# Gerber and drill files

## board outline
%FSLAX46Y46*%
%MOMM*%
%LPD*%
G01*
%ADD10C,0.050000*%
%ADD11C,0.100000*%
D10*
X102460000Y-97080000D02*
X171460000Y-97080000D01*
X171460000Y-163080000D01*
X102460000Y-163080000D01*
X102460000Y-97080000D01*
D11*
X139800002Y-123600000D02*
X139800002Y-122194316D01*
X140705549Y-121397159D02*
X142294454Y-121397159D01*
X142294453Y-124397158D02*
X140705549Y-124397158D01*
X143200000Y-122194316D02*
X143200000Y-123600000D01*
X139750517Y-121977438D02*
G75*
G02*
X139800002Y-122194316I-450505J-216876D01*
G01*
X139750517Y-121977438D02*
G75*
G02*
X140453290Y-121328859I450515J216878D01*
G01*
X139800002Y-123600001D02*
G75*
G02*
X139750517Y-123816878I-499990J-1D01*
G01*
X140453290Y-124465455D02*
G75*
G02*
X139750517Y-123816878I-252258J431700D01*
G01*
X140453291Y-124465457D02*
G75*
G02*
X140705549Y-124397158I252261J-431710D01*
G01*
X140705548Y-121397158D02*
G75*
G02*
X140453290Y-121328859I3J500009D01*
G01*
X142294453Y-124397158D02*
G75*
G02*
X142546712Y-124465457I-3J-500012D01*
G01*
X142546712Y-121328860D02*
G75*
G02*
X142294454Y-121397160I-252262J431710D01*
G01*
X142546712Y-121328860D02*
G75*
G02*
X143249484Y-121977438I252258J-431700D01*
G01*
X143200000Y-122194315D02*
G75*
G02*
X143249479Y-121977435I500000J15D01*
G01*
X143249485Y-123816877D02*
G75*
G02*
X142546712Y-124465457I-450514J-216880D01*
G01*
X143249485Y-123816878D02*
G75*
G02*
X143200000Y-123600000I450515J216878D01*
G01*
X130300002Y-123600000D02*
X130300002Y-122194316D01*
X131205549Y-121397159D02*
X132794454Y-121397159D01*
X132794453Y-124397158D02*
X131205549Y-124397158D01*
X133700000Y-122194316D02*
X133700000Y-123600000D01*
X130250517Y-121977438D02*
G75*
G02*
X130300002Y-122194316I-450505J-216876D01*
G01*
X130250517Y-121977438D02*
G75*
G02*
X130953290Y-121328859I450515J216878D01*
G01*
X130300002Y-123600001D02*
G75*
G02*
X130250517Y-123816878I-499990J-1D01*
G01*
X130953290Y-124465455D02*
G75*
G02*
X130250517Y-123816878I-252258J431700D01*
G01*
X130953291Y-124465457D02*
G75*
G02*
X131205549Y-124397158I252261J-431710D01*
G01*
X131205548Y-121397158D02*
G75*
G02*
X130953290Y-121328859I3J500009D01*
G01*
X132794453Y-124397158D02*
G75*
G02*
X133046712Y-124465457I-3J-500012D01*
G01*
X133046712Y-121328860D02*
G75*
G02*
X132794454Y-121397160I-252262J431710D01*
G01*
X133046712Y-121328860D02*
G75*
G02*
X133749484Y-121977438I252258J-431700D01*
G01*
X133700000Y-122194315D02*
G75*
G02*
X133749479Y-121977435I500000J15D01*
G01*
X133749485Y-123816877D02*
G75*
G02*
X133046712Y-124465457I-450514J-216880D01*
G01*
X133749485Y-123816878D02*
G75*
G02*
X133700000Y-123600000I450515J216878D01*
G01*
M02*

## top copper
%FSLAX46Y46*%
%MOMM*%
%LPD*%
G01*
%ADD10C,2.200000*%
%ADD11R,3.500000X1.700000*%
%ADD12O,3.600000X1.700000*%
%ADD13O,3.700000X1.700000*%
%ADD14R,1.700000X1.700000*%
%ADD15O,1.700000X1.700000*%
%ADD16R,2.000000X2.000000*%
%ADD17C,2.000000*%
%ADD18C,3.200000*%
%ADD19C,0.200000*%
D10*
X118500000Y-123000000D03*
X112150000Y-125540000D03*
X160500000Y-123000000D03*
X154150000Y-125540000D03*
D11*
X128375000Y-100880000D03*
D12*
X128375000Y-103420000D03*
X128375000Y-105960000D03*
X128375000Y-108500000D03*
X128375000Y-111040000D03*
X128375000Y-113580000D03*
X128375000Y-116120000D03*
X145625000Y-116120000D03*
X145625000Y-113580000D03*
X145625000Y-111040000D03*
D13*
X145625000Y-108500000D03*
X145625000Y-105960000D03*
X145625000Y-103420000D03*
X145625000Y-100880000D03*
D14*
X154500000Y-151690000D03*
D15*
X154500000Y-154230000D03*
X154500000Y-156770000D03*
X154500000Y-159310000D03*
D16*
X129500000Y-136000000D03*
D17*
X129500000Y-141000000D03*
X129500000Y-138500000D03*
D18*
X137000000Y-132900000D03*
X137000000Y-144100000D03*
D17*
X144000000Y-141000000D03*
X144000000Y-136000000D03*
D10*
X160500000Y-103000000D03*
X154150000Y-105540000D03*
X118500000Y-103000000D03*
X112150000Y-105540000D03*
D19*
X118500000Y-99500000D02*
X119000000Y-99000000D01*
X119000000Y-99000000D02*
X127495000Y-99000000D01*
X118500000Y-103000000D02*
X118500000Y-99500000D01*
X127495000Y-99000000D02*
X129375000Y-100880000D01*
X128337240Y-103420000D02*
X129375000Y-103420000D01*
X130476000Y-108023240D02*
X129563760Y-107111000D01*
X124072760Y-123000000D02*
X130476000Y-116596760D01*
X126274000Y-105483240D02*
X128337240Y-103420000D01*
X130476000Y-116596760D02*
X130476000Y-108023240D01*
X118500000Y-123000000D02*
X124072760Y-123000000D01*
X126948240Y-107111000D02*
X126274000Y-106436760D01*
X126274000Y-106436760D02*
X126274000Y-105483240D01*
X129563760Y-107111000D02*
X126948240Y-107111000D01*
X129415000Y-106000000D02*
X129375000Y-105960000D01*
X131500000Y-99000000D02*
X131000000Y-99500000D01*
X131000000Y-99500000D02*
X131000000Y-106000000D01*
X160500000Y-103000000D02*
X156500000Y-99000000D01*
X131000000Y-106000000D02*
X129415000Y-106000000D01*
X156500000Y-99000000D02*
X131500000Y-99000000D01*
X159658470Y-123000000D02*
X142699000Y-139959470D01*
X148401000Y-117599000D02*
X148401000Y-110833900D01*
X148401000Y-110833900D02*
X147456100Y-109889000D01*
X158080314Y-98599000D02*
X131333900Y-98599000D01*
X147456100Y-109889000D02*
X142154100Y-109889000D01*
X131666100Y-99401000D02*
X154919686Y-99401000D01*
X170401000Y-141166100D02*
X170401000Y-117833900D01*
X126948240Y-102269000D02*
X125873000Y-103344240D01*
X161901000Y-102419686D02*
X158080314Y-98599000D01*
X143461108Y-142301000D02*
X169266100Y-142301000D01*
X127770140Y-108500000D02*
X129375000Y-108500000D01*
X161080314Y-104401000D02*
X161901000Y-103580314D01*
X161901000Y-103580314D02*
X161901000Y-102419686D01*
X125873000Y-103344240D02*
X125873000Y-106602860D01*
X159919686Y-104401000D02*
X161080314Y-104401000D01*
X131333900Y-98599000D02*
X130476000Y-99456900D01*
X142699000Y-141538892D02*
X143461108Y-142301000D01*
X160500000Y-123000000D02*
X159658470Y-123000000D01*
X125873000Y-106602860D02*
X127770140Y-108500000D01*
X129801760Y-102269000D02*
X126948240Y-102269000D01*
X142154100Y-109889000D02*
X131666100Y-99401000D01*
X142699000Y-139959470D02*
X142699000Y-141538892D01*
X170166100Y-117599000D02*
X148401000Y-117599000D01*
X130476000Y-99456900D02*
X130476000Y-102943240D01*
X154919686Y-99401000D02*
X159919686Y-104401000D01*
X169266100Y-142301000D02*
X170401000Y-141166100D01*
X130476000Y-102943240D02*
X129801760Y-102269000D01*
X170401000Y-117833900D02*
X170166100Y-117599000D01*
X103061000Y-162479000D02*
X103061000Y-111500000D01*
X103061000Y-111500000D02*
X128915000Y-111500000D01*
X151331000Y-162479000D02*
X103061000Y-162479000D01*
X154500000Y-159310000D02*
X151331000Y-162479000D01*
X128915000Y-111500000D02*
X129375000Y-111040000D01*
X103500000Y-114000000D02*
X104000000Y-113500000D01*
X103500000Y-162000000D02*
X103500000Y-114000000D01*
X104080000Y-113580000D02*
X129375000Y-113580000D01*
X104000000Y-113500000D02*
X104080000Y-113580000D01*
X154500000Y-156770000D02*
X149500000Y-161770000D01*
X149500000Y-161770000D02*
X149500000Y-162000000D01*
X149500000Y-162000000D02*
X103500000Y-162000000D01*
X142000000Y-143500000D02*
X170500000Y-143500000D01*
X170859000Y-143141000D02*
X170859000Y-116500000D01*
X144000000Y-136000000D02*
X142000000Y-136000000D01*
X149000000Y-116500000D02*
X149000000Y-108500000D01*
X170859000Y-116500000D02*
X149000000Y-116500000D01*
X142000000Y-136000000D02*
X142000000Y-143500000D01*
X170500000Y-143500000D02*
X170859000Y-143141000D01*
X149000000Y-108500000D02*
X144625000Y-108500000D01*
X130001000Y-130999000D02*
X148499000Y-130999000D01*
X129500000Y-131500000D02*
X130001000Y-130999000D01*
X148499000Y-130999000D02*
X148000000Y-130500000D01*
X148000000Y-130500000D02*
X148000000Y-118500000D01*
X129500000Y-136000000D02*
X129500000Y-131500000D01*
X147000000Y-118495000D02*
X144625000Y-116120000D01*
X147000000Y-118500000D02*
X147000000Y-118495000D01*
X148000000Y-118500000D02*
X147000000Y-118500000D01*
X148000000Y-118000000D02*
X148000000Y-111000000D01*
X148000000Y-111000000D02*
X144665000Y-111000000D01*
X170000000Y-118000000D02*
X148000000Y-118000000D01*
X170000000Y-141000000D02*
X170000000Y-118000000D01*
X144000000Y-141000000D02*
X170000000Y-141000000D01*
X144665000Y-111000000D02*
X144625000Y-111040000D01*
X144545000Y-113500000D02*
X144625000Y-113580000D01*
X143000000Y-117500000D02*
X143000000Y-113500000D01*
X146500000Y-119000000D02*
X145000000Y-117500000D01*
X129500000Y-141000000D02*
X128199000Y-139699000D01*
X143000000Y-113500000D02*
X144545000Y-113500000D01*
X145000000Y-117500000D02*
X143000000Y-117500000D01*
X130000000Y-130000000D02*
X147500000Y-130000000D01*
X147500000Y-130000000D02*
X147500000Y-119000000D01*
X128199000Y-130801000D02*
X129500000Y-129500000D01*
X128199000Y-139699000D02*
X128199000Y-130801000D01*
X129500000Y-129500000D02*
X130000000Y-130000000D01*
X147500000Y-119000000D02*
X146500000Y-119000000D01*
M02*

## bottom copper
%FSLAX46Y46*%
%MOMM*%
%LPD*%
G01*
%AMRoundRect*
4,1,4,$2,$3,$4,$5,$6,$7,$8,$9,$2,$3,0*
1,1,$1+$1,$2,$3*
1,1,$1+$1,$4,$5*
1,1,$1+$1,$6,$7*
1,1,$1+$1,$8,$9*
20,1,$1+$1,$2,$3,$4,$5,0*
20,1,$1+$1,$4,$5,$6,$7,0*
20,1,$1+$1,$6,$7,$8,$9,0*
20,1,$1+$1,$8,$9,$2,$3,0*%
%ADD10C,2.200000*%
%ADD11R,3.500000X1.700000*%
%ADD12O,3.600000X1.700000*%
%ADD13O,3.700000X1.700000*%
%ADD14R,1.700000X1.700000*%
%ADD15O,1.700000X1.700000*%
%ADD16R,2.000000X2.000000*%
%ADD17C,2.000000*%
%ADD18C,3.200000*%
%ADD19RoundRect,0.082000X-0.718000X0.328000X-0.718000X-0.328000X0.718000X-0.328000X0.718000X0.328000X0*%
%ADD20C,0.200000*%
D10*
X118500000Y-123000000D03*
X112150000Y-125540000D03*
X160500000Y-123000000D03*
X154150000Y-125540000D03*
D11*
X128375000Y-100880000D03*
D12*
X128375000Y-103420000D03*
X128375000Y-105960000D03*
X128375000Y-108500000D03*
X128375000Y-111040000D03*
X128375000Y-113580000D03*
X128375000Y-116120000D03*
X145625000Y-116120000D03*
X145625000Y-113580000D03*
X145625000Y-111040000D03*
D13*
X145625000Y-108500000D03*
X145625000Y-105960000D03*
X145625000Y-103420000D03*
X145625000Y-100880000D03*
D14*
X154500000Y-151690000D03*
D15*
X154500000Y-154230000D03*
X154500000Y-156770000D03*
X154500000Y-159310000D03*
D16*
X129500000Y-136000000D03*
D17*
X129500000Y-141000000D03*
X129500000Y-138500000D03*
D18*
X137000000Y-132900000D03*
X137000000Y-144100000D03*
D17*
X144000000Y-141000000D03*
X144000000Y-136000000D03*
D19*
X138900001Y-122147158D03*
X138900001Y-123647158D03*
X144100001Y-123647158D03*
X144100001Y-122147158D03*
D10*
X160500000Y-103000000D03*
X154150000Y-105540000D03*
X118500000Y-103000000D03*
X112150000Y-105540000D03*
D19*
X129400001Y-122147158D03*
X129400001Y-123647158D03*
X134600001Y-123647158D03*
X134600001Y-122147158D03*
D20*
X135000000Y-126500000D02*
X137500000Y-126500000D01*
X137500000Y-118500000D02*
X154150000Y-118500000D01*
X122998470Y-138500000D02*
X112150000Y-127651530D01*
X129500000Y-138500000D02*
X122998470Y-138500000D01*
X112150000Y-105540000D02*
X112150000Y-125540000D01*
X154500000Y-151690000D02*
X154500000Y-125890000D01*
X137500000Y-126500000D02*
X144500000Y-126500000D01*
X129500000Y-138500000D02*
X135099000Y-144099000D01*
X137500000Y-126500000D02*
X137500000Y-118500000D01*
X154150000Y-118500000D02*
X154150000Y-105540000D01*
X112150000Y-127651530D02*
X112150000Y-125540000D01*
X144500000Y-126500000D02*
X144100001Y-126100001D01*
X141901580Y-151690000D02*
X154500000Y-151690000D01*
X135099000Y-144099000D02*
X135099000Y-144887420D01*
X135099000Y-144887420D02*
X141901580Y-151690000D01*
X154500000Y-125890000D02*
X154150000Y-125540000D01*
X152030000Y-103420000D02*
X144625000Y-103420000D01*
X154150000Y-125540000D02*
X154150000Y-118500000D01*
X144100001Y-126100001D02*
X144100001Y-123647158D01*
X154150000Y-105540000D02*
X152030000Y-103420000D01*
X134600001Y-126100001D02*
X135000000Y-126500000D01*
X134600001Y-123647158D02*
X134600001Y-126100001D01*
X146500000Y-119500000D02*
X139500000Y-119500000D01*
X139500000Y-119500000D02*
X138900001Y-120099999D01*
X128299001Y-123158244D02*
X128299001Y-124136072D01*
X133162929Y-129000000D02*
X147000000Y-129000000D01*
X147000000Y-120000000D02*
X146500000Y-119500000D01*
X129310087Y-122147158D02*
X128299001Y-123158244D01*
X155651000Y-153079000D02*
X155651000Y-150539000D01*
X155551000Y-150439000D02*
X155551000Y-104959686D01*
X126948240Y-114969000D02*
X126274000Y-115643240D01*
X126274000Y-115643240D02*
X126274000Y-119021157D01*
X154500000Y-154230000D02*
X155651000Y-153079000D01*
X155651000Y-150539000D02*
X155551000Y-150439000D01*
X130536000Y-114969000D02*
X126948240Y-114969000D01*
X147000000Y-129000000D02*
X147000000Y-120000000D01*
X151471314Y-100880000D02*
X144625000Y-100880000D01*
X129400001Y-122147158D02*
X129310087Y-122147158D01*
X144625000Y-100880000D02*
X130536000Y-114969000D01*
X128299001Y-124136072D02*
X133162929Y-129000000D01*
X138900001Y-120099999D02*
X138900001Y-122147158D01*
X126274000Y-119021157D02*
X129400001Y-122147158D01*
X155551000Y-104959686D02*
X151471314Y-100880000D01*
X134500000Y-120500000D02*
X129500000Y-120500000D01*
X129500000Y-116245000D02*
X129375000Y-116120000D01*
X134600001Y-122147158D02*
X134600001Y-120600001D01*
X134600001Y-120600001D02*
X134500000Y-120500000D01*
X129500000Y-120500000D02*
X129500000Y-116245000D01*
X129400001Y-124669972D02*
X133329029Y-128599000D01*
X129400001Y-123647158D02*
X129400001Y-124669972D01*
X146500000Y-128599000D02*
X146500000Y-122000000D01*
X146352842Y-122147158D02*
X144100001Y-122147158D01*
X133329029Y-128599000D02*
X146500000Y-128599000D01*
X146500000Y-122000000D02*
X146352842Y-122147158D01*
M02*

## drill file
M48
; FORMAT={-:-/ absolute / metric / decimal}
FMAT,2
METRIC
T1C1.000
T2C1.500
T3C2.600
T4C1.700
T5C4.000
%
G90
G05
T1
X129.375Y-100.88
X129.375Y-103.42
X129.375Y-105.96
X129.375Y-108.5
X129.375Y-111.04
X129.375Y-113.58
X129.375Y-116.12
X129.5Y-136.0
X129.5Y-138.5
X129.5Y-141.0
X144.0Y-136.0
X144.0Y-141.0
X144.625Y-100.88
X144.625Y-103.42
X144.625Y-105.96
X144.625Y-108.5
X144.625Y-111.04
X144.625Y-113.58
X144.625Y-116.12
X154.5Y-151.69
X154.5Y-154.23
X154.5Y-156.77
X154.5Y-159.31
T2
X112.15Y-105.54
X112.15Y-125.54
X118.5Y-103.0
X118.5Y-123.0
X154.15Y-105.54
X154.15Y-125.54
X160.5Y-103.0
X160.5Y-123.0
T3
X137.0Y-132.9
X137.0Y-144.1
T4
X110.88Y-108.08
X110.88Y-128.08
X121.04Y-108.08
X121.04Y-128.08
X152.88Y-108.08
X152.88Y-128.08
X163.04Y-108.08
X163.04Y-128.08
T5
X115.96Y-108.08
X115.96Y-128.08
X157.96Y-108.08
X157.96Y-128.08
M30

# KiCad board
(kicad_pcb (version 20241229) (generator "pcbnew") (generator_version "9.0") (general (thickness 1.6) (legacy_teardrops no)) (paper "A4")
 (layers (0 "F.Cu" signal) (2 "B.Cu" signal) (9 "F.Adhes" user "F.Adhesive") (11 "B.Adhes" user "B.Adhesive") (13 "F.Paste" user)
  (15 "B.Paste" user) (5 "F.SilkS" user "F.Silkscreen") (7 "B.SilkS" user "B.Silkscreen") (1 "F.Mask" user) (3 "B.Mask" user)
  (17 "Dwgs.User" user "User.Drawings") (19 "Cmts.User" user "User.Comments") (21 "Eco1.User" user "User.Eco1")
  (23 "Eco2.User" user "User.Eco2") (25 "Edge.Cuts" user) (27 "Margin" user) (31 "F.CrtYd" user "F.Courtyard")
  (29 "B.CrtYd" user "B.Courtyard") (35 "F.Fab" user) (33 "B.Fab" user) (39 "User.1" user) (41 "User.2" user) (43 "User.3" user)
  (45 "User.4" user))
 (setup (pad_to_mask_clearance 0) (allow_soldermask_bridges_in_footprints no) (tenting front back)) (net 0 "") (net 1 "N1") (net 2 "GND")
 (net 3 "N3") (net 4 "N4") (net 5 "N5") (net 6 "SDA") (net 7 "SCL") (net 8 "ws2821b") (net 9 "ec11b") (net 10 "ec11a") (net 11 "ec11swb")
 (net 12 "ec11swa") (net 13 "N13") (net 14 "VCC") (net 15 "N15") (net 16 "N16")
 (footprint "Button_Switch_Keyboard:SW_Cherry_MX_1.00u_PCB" (layer "F.Cu") (at 118.5 123)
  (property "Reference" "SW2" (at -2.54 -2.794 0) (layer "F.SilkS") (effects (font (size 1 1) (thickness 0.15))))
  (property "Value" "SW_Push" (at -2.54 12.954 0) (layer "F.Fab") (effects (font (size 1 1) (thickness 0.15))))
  (pad "" np_thru_hole circle (at -7.62 5.08) (size 1.7 1.7) (drill 1.7) (layers "*.Cu" "*.Mask"))
  (pad "" np_thru_hole circle (at -2.54 5.08) (size 4 4) (drill 4) (layers "*.Cu" "*.Mask"))
  (pad "" np_thru_hole circle (at 2.54 5.08) (size 1.7 1.7) (drill 1.7) (layers "*.Cu" "*.Mask"))
  (pad "1" thru_hole circle (at 0 0) (size 2.2 2.2) (drill 1.5) (layers "*.Cu" "*.Mask") (remove_unused_layers no) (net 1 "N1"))
  (pad "2" thru_hole circle (at -6.35 2.54) (size 2.2 2.2) (drill 1.5) (layers "*.Cu" "*.Mask") (remove_unused_layers no) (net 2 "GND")))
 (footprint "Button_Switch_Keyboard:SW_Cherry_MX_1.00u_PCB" (layer "F.Cu") (at 160.5 123)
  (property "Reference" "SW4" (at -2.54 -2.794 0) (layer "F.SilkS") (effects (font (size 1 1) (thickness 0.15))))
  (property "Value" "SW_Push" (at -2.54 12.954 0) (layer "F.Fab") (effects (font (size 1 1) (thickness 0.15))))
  (pad "" np_thru_hole circle (at -7.62 5.08) (size 1.7 1.7) (drill 1.7) (layers "*.Cu" "*.Mask"))
  (pad "" np_thru_hole circle (at -2.54 5.08) (size 4 4) (drill 4) (layers "*.Cu" "*.Mask"))
  (pad "" np_thru_hole circle (at 2.54 5.08) (size 1.7 1.7) (drill 1.7) (layers "*.Cu" "*.Mask"))
  (pad "1" thru_hole circle (at 0 0) (size 2.2 2.2) (drill 1.5) (layers "*.Cu" "*.Mask") (remove_unused_layers no) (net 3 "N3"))
  (pad "2" thru_hole circle (at -6.35 2.54) (size 2.2 2.2) (drill 1.5) (layers "*.Cu" "*.Mask") (remove_unused_layers no) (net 2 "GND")))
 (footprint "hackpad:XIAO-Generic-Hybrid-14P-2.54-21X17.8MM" (layer "F.Cu") (at 137 108.5)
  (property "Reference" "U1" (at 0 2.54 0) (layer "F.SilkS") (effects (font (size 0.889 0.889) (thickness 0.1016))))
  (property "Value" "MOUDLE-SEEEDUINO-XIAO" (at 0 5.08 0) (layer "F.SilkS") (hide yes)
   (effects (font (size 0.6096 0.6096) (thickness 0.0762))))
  (pad "1" thru_hole rect (at -7.625 -7.62) (size 3.5 1.7) (drill 1 (offset -1 0)) (layers "*.Cu" "*.Mask") (remove_unused_layers no)
   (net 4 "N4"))
  (pad "2" thru_hole oval (at -7.625 -5.08) (size 3.6 1.7) (drill 1 (offset -1 0)) (layers "*.Cu" "*.Mask") (remove_unused_layers no)
   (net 1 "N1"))
  (pad "3" thru_hole oval (at -7.625 -2.54) (size 3.6 1.7) (drill 1 (offset -1 0)) (layers "*.Cu" "*.Mask") (remove_unused_layers no)
   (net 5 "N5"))
  (pad "4" thru_hole oval (at -7.625 0) (size 3.6 1.7) (drill 1 (offset -1 0)) (layers "*.Cu" "*.Mask") (remove_unused_layers no)
   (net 3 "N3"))
  (pad "5" thru_hole oval (at -7.625 2.54) (size 3.6 1.7) (drill 1 (offset -1 0)) (layers "*.Cu" "*.Mask") (remove_unused_layers no)
   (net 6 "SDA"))
  (pad "6" thru_hole oval (at -7.625 5.08 180) (size 3.6 1.7) (drill 1 (offset 1 0)) (layers "*.Cu" "*.Mask") (remove_unused_layers no)
   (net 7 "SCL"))
  (pad "7" thru_hole oval (at -7.625 7.62) (size 3.6 1.7) (drill 1 (offset -1 0)) (layers "*.Cu" "*.Mask") (remove_unused_layers no)
   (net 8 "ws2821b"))
  (pad "8" thru_hole oval (at 7.625 7.62) (size 3.6 1.7) (drill 1 (offset 1 0)) (layers "*.Cu" "*.Mask") (remove_unused_layers no)
   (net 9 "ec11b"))
  (pad "9" thru_hole oval (at 7.625 5.08) (size 3.6 1.7) (drill 1 (offset 1 0)) (layers "*.Cu" "*.Mask") (remove_unused_layers no)
   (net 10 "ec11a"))
  (pad "10" thru_hole oval (at 7.625 2.54) (size 3.6 1.7) (drill 1 (offset 1 0)) (layers "*.Cu" "*.Mask") (remove_unused_layers no)
   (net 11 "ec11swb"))
  (pad "11" thru_hole oval (at 7.625 0) (size 3.7 1.7) (drill 1 (offset 1 0)) (layers "*.Cu" "*.Mask") (remove_unused_layers no)
   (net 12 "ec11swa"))
  (pad "12" thru_hole oval (at 7.625 -2.54) (size 3.7 1.7) (drill 1 (offset 1 0)) (layers "*.Cu" "*.Mask") (remove_unused_layers no)
   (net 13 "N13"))
  (pad "13" thru_hole oval (at 7.625 -5.08) (size 3.7 1.7) (drill 1 (offset 1 0)) (layers "*.Cu" "*.Mask") (remove_unused_layers no)
   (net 2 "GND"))
  (pad "14" thru_hole oval (at 7.625 -7.62) (size 3.7 1.7) (drill 1 (offset 1 0)) (layers "*.Cu" "*.Mask") (remove_unused_layers no)
   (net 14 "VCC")))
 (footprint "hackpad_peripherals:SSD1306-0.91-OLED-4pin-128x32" (layer "F.Cu") (at 118 149.5)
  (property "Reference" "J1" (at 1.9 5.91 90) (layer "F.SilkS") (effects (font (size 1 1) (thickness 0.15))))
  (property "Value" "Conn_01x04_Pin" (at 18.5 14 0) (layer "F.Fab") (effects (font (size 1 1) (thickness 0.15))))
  (pad "1" thru_hole rect (at 36.5 2.19) (size 1.7 1.7) (drill 1) (layers "*.Cu" "*.Mask") (remove_unused_layers no) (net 2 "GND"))
  (pad "2" thru_hole oval (at 36.5 4.73) (size 1.7 1.7) (drill 1) (layers "*.Cu" "*.Mask") (remove_unused_layers no) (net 14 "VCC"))
  (pad "3" thru_hole oval (at 36.5 7.27) (size 1.7 1.7) (drill 1) (layers "*.Cu" "*.Mask") (remove_unused_layers no) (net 7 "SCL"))
  (pad "4" thru_hole oval (at 36.5 9.81) (size 1.7 1.7) (drill 1) (layers "*.Cu" "*.Mask") (remove_unused_layers no) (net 6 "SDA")))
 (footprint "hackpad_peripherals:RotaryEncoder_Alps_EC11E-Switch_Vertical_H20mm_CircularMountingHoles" (layer "F.Cu") (at 129.5 136)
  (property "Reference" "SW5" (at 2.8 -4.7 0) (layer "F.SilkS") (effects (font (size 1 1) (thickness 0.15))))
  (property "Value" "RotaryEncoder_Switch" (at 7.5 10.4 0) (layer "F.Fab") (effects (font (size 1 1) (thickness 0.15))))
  (pad "A" thru_hole rect (at 0 0) (size 2 2) (drill 1) (layers "*.Cu" "*.Mask") (remove_unused_layers no) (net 9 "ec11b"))
  (pad "B" thru_hole circle (at 0 5) (size 2 2) (drill 1) (layers "*.Cu" "*.Mask") (remove_unused_layers no) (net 10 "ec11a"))
  (pad "C" thru_hole circle (at 0 2.5) (size 2 2) (drill 1) (layers "*.Cu" "*.Mask") (remove_unused_layers no) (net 2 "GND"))
  (pad "MP" thru_hole circle (at 7.5 -3.1) (size 3.2 3.2) (drill 2.6) (layers "*.Cu" "*.Mask") (remove_unused_layers no))
  (pad "MP" thru_hole circle (at 7.5 8.1) (size 3.2 3.2) (drill 2.6) (layers "*.Cu" "*.Mask") (remove_unused_layers no))
  (pad "S1" thru_hole circle (at 14.5 5) (size 2 2) (drill 1) (layers "*.Cu" "*.Mask") (remove_unused_layers no) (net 11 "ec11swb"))
  (pad "S2" thru_hole circle (at 14.5 0) (size 2 2) (drill 1) (layers "*.Cu" "*.Mask") (remove_unused_layers no) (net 12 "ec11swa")))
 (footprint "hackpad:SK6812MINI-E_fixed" (layer "F.Cu") (at 141.5 123)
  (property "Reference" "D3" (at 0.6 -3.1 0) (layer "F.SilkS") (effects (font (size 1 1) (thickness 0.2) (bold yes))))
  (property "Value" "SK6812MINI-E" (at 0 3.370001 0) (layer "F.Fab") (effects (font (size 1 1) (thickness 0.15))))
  (fp_line (start -1.699998 0.6) (end -1.699998 -0.805684) (stroke (width 0.1) (type solid)) (layer "Edge.Cuts"))
  (fp_line (start -0.794451 -1.602841) (end 0.794454 -1.602841) (stroke (width 0.1) (type solid)) (layer "Edge.Cuts"))
  (fp_line (start 0.794453 1.397158) (end -0.794451 1.397158) (stroke (width 0.1) (type solid)) (layer "Edge.Cuts"))
  (fp_line (start 1.7 -0.805684) (end 1.7 0.6) (stroke (width 0.1) (type solid)) (layer "Edge.Cuts"))
  (fp_arc (start -1.749483 -1.022562) (mid -1.712526 -0.91691) (end -1.699998 -0.805684) (stroke (width 0.1) (type solid))
   (layer "Edge.Cuts"))
  (fp_arc (start -1.749483 -1.022562) (mid -1.63807 -1.606877) (end -1.04671 -1.671141) (stroke (width 0.1) (type solid))
   (layer "Edge.Cuts"))
  (fp_arc (start -1.699998 0.600001) (mid -1.712526 0.711226) (end -1.749483 0.816878) (stroke (width 0.1) (type solid)) (layer "Edge.Cuts"))
  (fp_arc (start -1.04671 1.465455) (mid -1.638069 1.401192) (end -1.749483 0.816878) (stroke (width 0.1) (type solid)) (layer "Edge.Cuts"))
  (fp_arc (start -1.046709 1.465457) (mid -0.925121 1.414535) (end -0.794451 1.397158) (stroke (width 0.1) (type solid)) (layer "Edge.Cuts"))
  (fp_arc (start -0.794452 -1.602842) (mid -0.925122 -1.620219) (end -1.04671 -1.671141) (stroke (width 0.1) (type solid))
   (layer "Edge.Cuts"))
  (fp_arc (start 0.794453 1.397158) (mid 0.925124 1.414535) (end 1.046712 1.465457) (stroke (width 0.1) (type solid)) (layer "Edge.Cuts"))
  (fp_arc (start 1.046712 -1.67114) (mid 0.925124 -1.620218) (end 0.794454 -1.602841) (stroke (width 0.1) (type solid)) (layer "Edge.Cuts"))
  (fp_arc (start 1.046712 -1.67114) (mid 1.638072 -1.606876) (end 1.749485 -1.022562) (stroke (width 0.1) (type solid)) (layer "Edge.Cuts"))
  (fp_arc (start 1.7 -0.805685) (mid 1.712528 -0.91691) (end 1.749485 -1.022562) (stroke (width 0.1) (type solid)) (layer "Edge.Cuts"))
  (fp_arc (start 1.749485 0.816877) (mid 1.638073 1.401193) (end 1.046712 1.465457) (stroke (width 0.1) (type solid)) (layer "Edge.Cuts"))
  (fp_arc (start 1.749485 0.816878) (mid 1.712528 0.711226) (end 1.7 0.6) (stroke (width 0.1) (type solid)) (layer "Edge.Cuts"))
  (pad "1" smd roundrect (at -2.599999 -0.852842 270) (size 0.82 1.6) (layers "B.Cu" "B.Mask" "B.Paste") (roundrect_rratio 0.1)
   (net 14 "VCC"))
  (pad "2" smd roundrect (at -2.599999 0.647158 270) (size 0.82 1.6) (layers "B.Cu" "B.Mask" "B.Paste") (roundrect_rratio 0.1)
   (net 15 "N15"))
  (pad "3" smd roundrect (at 2.600001 0.647158 270) (size 0.82 1.6) (layers "B.Cu" "B.Mask" "B.Paste") (roundrect_rratio 0.1) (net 2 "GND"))
  (pad "4" smd roundrect (at 2.600001 -0.852842 270) (size 0.82 1.6) (layers "B.Cu" "B.Mask" "B.Paste") (roundrect_rratio 0.1)
   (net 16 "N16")))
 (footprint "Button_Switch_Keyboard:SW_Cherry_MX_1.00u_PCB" (layer "F.Cu") (at 160.5 103)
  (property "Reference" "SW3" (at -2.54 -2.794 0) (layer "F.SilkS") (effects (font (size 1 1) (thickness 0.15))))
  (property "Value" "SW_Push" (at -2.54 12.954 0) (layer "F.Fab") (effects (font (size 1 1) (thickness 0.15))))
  (pad "" np_thru_hole circle (at -7.62 5.08) (size 1.7 1.7) (drill 1.7) (layers "*.Cu" "*.Mask"))
  (pad "" np_thru_hole circle (at -2.54 5.08) (size 4 4) (drill 4) (layers "*.Cu" "*.Mask"))
  (pad "" np_thru_hole circle (at 2.54 5.08) (size 1.7 1.7) (drill 1.7) (layers "*.Cu" "*.Mask"))
  (pad "1" thru_hole circle (at 0 0) (size 2.2 2.2) (drill 1.5) (layers "*.Cu" "*.Mask") (remove_unused_layers no) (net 5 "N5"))
  (pad "2" thru_hole circle (at -6.35 2.54) (size 2.2 2.2) (drill 1.5) (layers "*.Cu" "*.Mask") (remove_unused_layers no) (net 2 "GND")))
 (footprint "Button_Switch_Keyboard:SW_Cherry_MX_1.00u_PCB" (layer "F.Cu") (at 118.5 103)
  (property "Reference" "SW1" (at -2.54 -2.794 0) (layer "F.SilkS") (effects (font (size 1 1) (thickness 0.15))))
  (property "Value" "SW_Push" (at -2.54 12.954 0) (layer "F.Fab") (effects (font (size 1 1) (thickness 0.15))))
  (pad "" np_thru_hole circle (at -7.62 5.08) (size 1.7 1.7) (drill 1.7) (layers "*.Cu" "*.Mask"))
  (pad "" np_thru_hole circle (at -2.54 5.08) (size 4 4) (drill 4) (layers "*.Cu" "*.Mask"))
  (pad "" np_thru_hole circle (at 2.54 5.08) (size 1.7 1.7) (drill 1.7) (layers "*.Cu" "*.Mask"))
  (pad "1" thru_hole circle (at 0 0) (size 2.2 2.2) (drill 1.5) (layers "*.Cu" "*.Mask") (remove_unused_layers no) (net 4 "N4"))
  (pad "2" thru_hole circle (at -6.35 2.54) (size 2.2 2.2) (drill 1.5) (layers "*.Cu" "*.Mask") (remove_unused_layers no) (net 2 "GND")))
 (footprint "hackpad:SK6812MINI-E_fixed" (layer "F.Cu") (at 132 123)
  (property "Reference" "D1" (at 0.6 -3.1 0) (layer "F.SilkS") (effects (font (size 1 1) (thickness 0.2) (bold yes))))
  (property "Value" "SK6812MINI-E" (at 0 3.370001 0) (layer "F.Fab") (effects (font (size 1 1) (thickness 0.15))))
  (fp_line (start -1.699998 0.6) (end -1.699998 -0.805684) (stroke (width 0.1) (type solid)) (layer "Edge.Cuts"))
  (fp_line (start -0.794451 -1.602841) (end 0.794454 -1.602841) (stroke (width 0.1) (type solid)) (layer "Edge.Cuts"))
  (fp_line (start 0.794453 1.397158) (end -0.794451 1.397158) (stroke (width 0.1) (type solid)) (layer "Edge.Cuts"))
  (fp_line (start 1.7 -0.805684) (end 1.7 0.6) (stroke (width 0.1) (type solid)) (layer "Edge.Cuts"))
  (fp_arc (start -1.749483 -1.022562) (mid -1.712526 -0.91691) (end -1.699998 -0.805684) (stroke (width 0.1) (type solid))
   (layer "Edge.Cuts"))
  (fp_arc (start -1.749483 -1.022562) (mid -1.63807 -1.606877) (end -1.04671 -1.671141) (stroke (width 0.1) (type solid))
   (layer "Edge.Cuts"))
  (fp_arc (start -1.699998 0.600001) (mid -1.712526 0.711226) (end -1.749483 0.816878) (stroke (width 0.1) (type solid)) (layer "Edge.Cuts"))
  (fp_arc (start -1.04671 1.465455) (mid -1.638069 1.401192) (end -1.749483 0.816878) (stroke (width 0.1) (type solid)) (layer "Edge.Cuts"))
  (fp_arc (start -1.046709 1.465457) (mid -0.925121 1.414535) (end -0.794451 1.397158) (stroke (width 0.1) (type solid)) (layer "Edge.Cuts"))
  (fp_arc (start -0.794452 -1.602842) (mid -0.925122 -1.620219) (end -1.04671 -1.671141) (stroke (width 0.1) (type solid))
   (layer "Edge.Cuts"))
  (fp_arc (start 0.794453 1.397158) (mid 0.925124 1.414535) (end 1.046712 1.465457) (stroke (width 0.1) (type solid)) (layer "Edge.Cuts"))
  (fp_arc (start 1.046712 -1.67114) (mid 0.925124 -1.620218) (end 0.794454 -1.602841) (stroke (width 0.1) (type solid)) (layer "Edge.Cuts"))
  (fp_arc (start 1.046712 -1.67114) (mid 1.638072 -1.606876) (end 1.749485 -1.022562) (stroke (width 0.1) (type solid)) (layer "Edge.Cuts"))
  (fp_arc (start 1.7 -0.805685) (mid 1.712528 -0.91691) (end 1.749485 -1.022562) (stroke (width 0.1) (type solid)) (layer "Edge.Cuts"))
  (fp_arc (start 1.749485 0.816877) (mid 1.638073 1.401193) (end 1.046712 1.465457) (stroke (width 0.1) (type solid)) (layer "Edge.Cuts"))
  (fp_arc (start 1.749485 0.816878) (mid 1.712528 0.711226) (end 1.7 0.6) (stroke (width 0.1) (type solid)) (layer "Edge.Cuts"))
  (pad "1" smd roundrect (at -2.599999 -0.852842 270) (size 0.82 1.6) (layers "B.Cu" "B.Mask" "B.Paste") (roundrect_rratio 0.1)
   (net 14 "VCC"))
  (pad "2" smd roundrect (at -2.599999 0.647158 270) (size 0.82 1.6) (layers "B.Cu" "B.Mask" "B.Paste") (roundrect_rratio 0.1)
   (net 16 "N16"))
  (pad "3" smd roundrect (at 2.600001 0.647158 270) (size 0.82 1.6) (layers "B.Cu" "B.Mask" "B.Paste") (roundrect_rratio 0.1) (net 2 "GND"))
  (pad "4" smd roundrect (at 2.600001 -0.852842 270) (size 0.82 1.6) (layers "B.Cu" "B.Mask" "B.Paste") (roundrect_rratio 0.1)
   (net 8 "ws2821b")))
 (gr_rect (start 102.46 97.08) (end 171.46 163.08) (stroke (width 0.05) (type default)) (fill no) (layer "Edge.Cuts"))
 (segment (start 118.5 99.5) (end 119 99) (width 0.2) (layer "F.Cu") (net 4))
 (segment (start 119 99) (end 127.495 99) (width 0.2) (layer "F.Cu") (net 4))
 (segment (start 118.5 103) (end 118.5 99.5) (width 0.2) (layer "F.Cu") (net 4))
 (segment (start 127.495 99) (end 129.375 100.88) (width 0.2) (layer "F.Cu") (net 4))
 (segment (start 135 126.5) (end 137.5 126.5) (width 0.2) (layer "B.Cu") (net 2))
 (segment (start 137.5 118.5) (end 154.15 118.5) (width 0.2) (layer "B.Cu") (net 2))
 (segment (start 122.99847 138.5) (end 112.15 127.65153) (width 0.2) (layer "B.Cu") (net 2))
 (segment (start 129.5 138.5) (end 122.99847 138.5) (width 0.2) (layer "B.Cu") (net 2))
 (segment (start 112.15 105.54) (end 112.15 125.54) (width 0.2) (layer "B.Cu") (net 2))
 (segment (start 154.5 151.69) (end 154.5 125.89) (width 0.2) (layer "B.Cu") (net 2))
 (segment (start 137.5 126.5) (end 144.5 126.5) (width 0.2) (layer "B.Cu") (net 2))
 (segment (start 129.5 138.5) (end 135.099 144.099) (width 0.2) (layer "B.Cu") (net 2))
 (segment (start 137.5 126.5) (end 137.5 118.5) (width 0.2) (layer "B.Cu") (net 2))
 (segment (start 154.15 118.5) (end 154.15 105.54) (width 0.2) (layer "B.Cu") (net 2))
 (segment (start 112.15 127.65153) (end 112.15 125.54) (width 0.2) (layer "B.Cu") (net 2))
 (segment (start 144.5 126.5) (end 144.100001 126.100001) (width 0.2) (layer "B.Cu") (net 2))
 (segment (start 141.90158 151.69) (end 154.5 151.69) (width 0.2) (layer "B.Cu") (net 2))
 (segment (start 135.099 144.099) (end 135.099 144.88742) (width 0.2) (layer "B.Cu") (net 2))
 (segment (start 135.099 144.88742) (end 141.90158 151.69) (width 0.2) (layer "B.Cu") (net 2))
 (segment (start 154.5 125.89) (end 154.15 125.54) (width 0.2) (layer "B.Cu") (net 2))
 (segment (start 152.03 103.42) (end 144.625 103.42) (width 0.2) (layer "B.Cu") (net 2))
 (segment (start 154.15 125.54) (end 154.15 118.5) (width 0.2) (layer "B.Cu") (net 2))
 (segment (start 144.100001 126.100001) (end 144.100001 123.647158) (width 0.2) (layer "B.Cu") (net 2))
 (segment (start 154.15 105.54) (end 152.03 103.42) (width 0.2) (layer "B.Cu") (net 2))
 (segment (start 134.600001 126.100001) (end 135 126.5) (width 0.2) (layer "B.Cu") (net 2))
 (segment (start 134.600001 123.647158) (end 134.600001 126.100001) (width 0.2) (layer "B.Cu") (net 2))
 (segment (start 128.33724 103.42) (end 129.375 103.42) (width 0.2) (layer "F.Cu") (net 1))
 (segment (start 130.476 108.02324) (end 129.56376 107.111) (width 0.2) (layer "F.Cu") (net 1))
 (segment (start 124.07276 123) (end 130.476 116.59676) (width 0.2) (layer "F.Cu") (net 1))
 (segment (start 126.274 105.48324) (end 128.33724 103.42) (width 0.2) (layer "F.Cu") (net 1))
 (segment (start 130.476 116.59676) (end 130.476 108.02324) (width 0.2) (layer "F.Cu") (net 1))
 (segment (start 118.5 123) (end 124.07276 123) (width 0.2) (layer "F.Cu") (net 1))
 (segment (start 126.94824 107.111) (end 126.274 106.43676) (width 0.2) (layer "F.Cu") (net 1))
 (segment (start 126.274 106.43676) (end 126.274 105.48324) (width 0.2) (layer "F.Cu") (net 1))
 (segment (start 129.56376 107.111) (end 126.94824 107.111) (width 0.2) (layer "F.Cu") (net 1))
 (segment (start 129.415 106) (end 129.375 105.96) (width 0.2) (layer "F.Cu") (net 5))
 (segment (start 131.5 99) (end 131 99.5) (width 0.2) (layer "F.Cu") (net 5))
 (segment (start 131 99.5) (end 131 106) (width 0.2) (layer "F.Cu") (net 5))
 (segment (start 160.5 103) (end 156.5 99) (width 0.2) (layer "F.Cu") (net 5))
 (segment (start 131 106) (end 129.415 106) (width 0.2) (layer "F.Cu") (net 5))
 (segment (start 156.5 99) (end 131.5 99) (width 0.2) (layer "F.Cu") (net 5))
 (segment (start 159.65847 123) (end 142.699 139.95947) (width 0.2) (layer "F.Cu") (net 3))
 (segment (start 148.401 117.599) (end 148.401 110.8339) (width 0.2) (layer "F.Cu") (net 3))
 (segment (start 148.401 110.8339) (end 147.4561 109.889) (width 0.2) (layer "F.Cu") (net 3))
 (segment (start 158.080314 98.599) (end 131.3339 98.599) (width 0.2) (layer "F.Cu") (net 3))
 (segment (start 147.4561 109.889) (end 142.1541 109.889) (width 0.2) (layer "F.Cu") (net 3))
 (segment (start 131.6661 99.401) (end 154.919686 99.401) (width 0.2) (layer "F.Cu") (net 3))
 (segment (start 170.401 141.1661) (end 170.401 117.8339) (width 0.2) (layer "F.Cu") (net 3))
 (segment (start 126.94824 102.269) (end 125.873 103.34424) (width 0.2) (layer "F.Cu") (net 3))
 (segment (start 161.901 102.419686) (end 158.080314 98.599) (width 0.2) (layer "F.Cu") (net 3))
 (segment (start 143.461108 142.301) (end 169.2661 142.301) (width 0.2) (layer "F.Cu") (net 3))
 (segment (start 127.77014 108.5) (end 129.375 108.5) (width 0.2) (layer "F.Cu") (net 3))
 (segment (start 161.080314 104.401) (end 161.901 103.580314) (width 0.2) (layer "F.Cu") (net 3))
 (segment (start 161.901 103.580314) (end 161.901 102.419686) (width 0.2) (layer "F.Cu") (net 3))
 (segment (start 125.873 103.34424) (end 125.873 106.60286) (width 0.2) (layer "F.Cu") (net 3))
 (segment (start 159.919686 104.401) (end 161.080314 104.401) (width 0.2) (layer "F.Cu") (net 3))
 (segment (start 131.3339 98.599) (end 130.476 99.4569) (width 0.2) (layer "F.Cu") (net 3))
 (segment (start 142.699 141.538892) (end 143.461108 142.301) (width 0.2) (layer "F.Cu") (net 3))
 (segment (start 160.5 123) (end 159.65847 123) (width 0.2) (layer "F.Cu") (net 3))
 (segment (start 125.873 106.60286) (end 127.77014 108.5) (width 0.2) (layer "F.Cu") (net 3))
 (segment (start 129.80176 102.269) (end 126.94824 102.269) (width 0.2) (layer "F.Cu") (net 3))
 (segment (start 142.1541 109.889) (end 131.6661 99.401) (width 0.2) (layer "F.Cu") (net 3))
 (segment (start 142.699 139.95947) (end 142.699 141.538892) (width 0.2) (layer "F.Cu") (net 3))
 (segment (start 170.1661 117.599) (end 148.401 117.599) (width 0.2) (layer "F.Cu") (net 3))
 (segment (start 130.476 99.4569) (end 130.476 102.94324) (width 0.2) (layer "F.Cu") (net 3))
 (segment (start 154.919686 99.401) (end 159.919686 104.401) (width 0.2) (layer "F.Cu") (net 3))
 (segment (start 169.2661 142.301) (end 170.401 141.1661) (width 0.2) (layer "F.Cu") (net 3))
 (segment (start 130.476 102.94324) (end 129.80176 102.269) (width 0.2) (layer "F.Cu") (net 3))
 (segment (start 170.401 117.8339) (end 170.1661 117.599) (width 0.2) (layer "F.Cu") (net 3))
 (segment (start 146.5 119.5) (end 139.5 119.5) (width 0.2) (layer "B.Cu") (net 14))
 (segment (start 139.5 119.5) (end 138.900001 120.099999) (width 0.2) (layer "B.Cu") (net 14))
 (segment (start 128.299001 123.158244) (end 128.299001 124.136072) (width 0.2) (layer "B.Cu") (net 14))
 (segment (start 133.162929 129) (end 147 129) (width 0.2) (layer "B.Cu") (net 14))
 (segment (start 147 120) (end 146.5 119.5) (width 0.2) (layer "B.Cu") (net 14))
 (segment (start 129.310087 122.147158) (end 128.299001 123.158244) (width 0.2) (layer "B.Cu") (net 14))
 (segment (start 155.651 153.079) (end 155.651 150.539) (width 0.2) (layer "B.Cu") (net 14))
 (segment (start 155.551 150.439) (end 155.551 104.959686) (width 0.2) (layer "B.Cu") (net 14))
 (segment (start 126.94824 114.969) (end 126.274 115.64324) (width 0.2) (layer "B.Cu") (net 14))
 (segment (start 126.274 115.64324) (end 126.274 119.021157) (width 0.2) (layer "B.Cu") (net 14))
 (segment (start 154.5 154.23) (end 155.651 153.079) (width 0.2) (layer "B.Cu") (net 14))
 (segment (start 155.651 150.539) (end 155.551 150.439) (width 0.2) (layer "B.Cu") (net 14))
 (segment (start 130.536 114.969) (end 126.94824 114.969) (width 0.2) (layer "B.Cu") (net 14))
 (segment (start 147 129) (end 147 120) (width 0.2) (layer "B.Cu") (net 14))
 (segment (start 151.471314 100.88) (end 144.625 100.88) (width 0.2) (layer "B.Cu") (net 14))
 (segment (start 129.400001 122.147158) (end 129.310087 122.147158) (width 0.2) (layer "B.Cu") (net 14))
 (segment (start 144.625 100.88) (end 130.536 114.969) (width 0.2) (layer "B.Cu") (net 14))
 (segment (start 128.299001 124.136072) (end 133.162929 129) (width 0.2) (layer "B.Cu") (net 14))
 (segment (start 138.900001 120.099999) (end 138.900001 122.147158) (width 0.2) (layer "B.Cu") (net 14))
 (segment (start 126.274 119.021157) (end 129.400001 122.147158) (width 0.2) (layer "B.Cu") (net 14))
 (segment (start 155.551 104.959686) (end 151.471314 100.88) (width 0.2) (layer "B.Cu") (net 14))
 (segment (start 134.5 120.5) (end 129.5 120.5) (width 0.2) (layer "B.Cu") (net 8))
 (segment (start 129.5 116.245) (end 129.375 116.12) (width 0.2) (layer "B.Cu") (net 8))
 (segment (start 134.600001 122.147158) (end 134.600001 120.600001) (width 0.2) (layer "B.Cu") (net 8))
 (segment (start 134.600001 120.600001) (end 134.5 120.5) (width 0.2) (layer "B.Cu") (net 8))
 (segment (start 129.5 120.5) (end 129.5 116.245) (width 0.2) (layer "B.Cu") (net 8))
 (segment (start 103.061 162.479) (end 103.061 111.5) (width 0.2) (layer "F.Cu") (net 6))
 (segment (start 103.061 111.5) (end 128.915 111.5) (width 0.2) (layer "F.Cu") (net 6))
 (segment (start 151.331 162.479) (end 103.061 162.479) (width 0.2) (layer "F.Cu") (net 6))
 (segment (start 154.5 159.31) (end 151.331 162.479) (width 0.2) (layer "F.Cu") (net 6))
 (segment (start 128.915 111.5) (end 129.375 111.04) (width 0.2) (layer "F.Cu") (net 6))
 (segment (start 103.5 114) (end 104 113.5) (width 0.2) (layer "F.Cu") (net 7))
 (segment (start 103.5 162) (end 103.5 114) (width 0.2) (layer "F.Cu") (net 7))
 (segment (start 104.08 113.58) (end 129.375 113.58) (width 0.2) (layer "F.Cu") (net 7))
 (segment (start 104 113.5) (end 104.08 113.58) (width 0.2) (layer "F.Cu") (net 7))
 (segment (start 154.5 156.77) (end 149.5 161.77) (width 0.2) (layer "F.Cu") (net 7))
 (segment (start 149.5 161.77) (end 149.5 162) (width 0.2) (layer "F.Cu") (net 7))
 (segment (start 149.5 162) (end 103.5 162) (width 0.2) (layer "F.Cu") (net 7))
 (segment (start 142 143.5) (end 170.5 143.5) (width 0.2) (layer "F.Cu") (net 12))
 (segment (start 170.859 143.141) (end 170.859 116.5) (width 0.2) (layer "F.Cu") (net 12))
 (segment (start 144 136) (end 142 136) (width 0.2) (layer "F.Cu") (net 12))
 (segment (start 149 116.5) (end 149 108.5) (width 0.2) (layer "F.Cu") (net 12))
 (segment (start 170.859 116.5) (end 149 116.5) (width 0.2) (layer "F.Cu") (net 12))
 (segment (start 142 136) (end 142 143.5) (width 0.2) (layer "F.Cu") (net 12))
 (segment (start 170.5 143.5) (end 170.859 143.141) (width 0.2) (layer "F.Cu") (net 12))
 (segment (start 149 108.5) (end 144.625 108.5) (width 0.2) (layer "F.Cu") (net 12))
 (segment (start 130.001 130.999) (end 148.499 130.999) (width 0.2) (layer "F.Cu") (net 9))
 (segment (start 129.5 131.5) (end 130.001 130.999) (width 0.2) (layer "F.Cu") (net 9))
 (segment (start 148.499 130.999) (end 148 130.5) (width 0.2) (layer "F.Cu") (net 9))
 (segment (start 148 130.5) (end 148 118.5) (width 0.2) (layer "F.Cu") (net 9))
 (segment (start 129.5 136) (end 129.5 131.5) (width 0.2) (layer "F.Cu") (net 9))
 (segment (start 147 118.495) (end 144.625 116.12) (width 0.2) (layer "F.Cu") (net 9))
 (segment (start 147 118.5) (end 147 118.495) (width 0.2) (layer "F.Cu") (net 9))
 (segment (start 148 118.5) (end 147 118.5) (width 0.2) (layer "F.Cu") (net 9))
 (segment (start 148 118) (end 148 111) (width 0.2) (layer "F.Cu") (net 11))
 (segment (start 148 111) (end 144.665 111) (width 0.2) (layer "F.Cu") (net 11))
 (segment (start 170 118) (end 148 118) (width 0.2) (layer "F.Cu") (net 11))
 (segment (start 170 141) (end 170 118) (width 0.2) (layer "F.Cu") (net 11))
 (segment (start 144 141) (end 170 141) (width 0.2) (layer "F.Cu") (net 11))
 (segment (start 144.665 111) (end 144.625 111.04) (width 0.2) (layer "F.Cu") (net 11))
 (segment (start 144.545 113.5) (end 144.625 113.58) (width 0.2) (layer "F.Cu") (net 10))
 (segment (start 143 117.5) (end 143 113.5) (width 0.2) (layer "F.Cu") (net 10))
 (segment (start 146.5 119) (end 145 117.5) (width 0.2) (layer "F.Cu") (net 10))
 (segment (start 129.5 141) (end 128.199 139.699) (width 0.2) (layer "F.Cu") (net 10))
 (segment (start 143 113.5) (end 144.545 113.5) (width 0.2) (layer "F.Cu") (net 10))
 (segment (start 145 117.5) (end 143 117.5) (width 0.2) (layer "F.Cu") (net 10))
 (segment (start 130 130) (end 147.5 130) (width 0.2) (layer "F.Cu") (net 10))
 (segment (start 147.5 130) (end 147.5 119) (width 0.2) (layer "F.Cu") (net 10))
 (segment (start 128.199 130.801) (end 129.5 129.5) (width 0.2) (layer "F.Cu") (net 10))
 (segment (start 128.199 139.699) (end 128.199 130.801) (width 0.2) (layer "F.Cu") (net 10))
 (segment (start 129.5 129.5) (end 130 130) (width 0.2) (layer "F.Cu") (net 10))
 (segment (start 147.5 119) (end 146.5 119) (width 0.2) (layer "F.Cu") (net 10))
 (segment (start 129.400001 124.669972) (end 133.329029 128.599) (width 0.2) (layer "B.Cu") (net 16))
 (segment (start 129.400001 123.647158) (end 129.400001 124.669972) (width 0.2) (layer "B.Cu") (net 16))
 (segment (start 146.5 128.599) (end 146.5 122) (width 0.2) (layer "B.Cu") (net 16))
 (segment (start 146.352842 122.147158) (end 144.100001 122.147158) (width 0.2) (layer "B.Cu") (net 16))
 (segment (start 133.329029 128.599) (end 146.5 128.599) (width 0.2) (layer "B.Cu") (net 16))
 (segment (start 146.5 122) (end 146.352842 122.147158) (width 0.2) (layer "B.Cu") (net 16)))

